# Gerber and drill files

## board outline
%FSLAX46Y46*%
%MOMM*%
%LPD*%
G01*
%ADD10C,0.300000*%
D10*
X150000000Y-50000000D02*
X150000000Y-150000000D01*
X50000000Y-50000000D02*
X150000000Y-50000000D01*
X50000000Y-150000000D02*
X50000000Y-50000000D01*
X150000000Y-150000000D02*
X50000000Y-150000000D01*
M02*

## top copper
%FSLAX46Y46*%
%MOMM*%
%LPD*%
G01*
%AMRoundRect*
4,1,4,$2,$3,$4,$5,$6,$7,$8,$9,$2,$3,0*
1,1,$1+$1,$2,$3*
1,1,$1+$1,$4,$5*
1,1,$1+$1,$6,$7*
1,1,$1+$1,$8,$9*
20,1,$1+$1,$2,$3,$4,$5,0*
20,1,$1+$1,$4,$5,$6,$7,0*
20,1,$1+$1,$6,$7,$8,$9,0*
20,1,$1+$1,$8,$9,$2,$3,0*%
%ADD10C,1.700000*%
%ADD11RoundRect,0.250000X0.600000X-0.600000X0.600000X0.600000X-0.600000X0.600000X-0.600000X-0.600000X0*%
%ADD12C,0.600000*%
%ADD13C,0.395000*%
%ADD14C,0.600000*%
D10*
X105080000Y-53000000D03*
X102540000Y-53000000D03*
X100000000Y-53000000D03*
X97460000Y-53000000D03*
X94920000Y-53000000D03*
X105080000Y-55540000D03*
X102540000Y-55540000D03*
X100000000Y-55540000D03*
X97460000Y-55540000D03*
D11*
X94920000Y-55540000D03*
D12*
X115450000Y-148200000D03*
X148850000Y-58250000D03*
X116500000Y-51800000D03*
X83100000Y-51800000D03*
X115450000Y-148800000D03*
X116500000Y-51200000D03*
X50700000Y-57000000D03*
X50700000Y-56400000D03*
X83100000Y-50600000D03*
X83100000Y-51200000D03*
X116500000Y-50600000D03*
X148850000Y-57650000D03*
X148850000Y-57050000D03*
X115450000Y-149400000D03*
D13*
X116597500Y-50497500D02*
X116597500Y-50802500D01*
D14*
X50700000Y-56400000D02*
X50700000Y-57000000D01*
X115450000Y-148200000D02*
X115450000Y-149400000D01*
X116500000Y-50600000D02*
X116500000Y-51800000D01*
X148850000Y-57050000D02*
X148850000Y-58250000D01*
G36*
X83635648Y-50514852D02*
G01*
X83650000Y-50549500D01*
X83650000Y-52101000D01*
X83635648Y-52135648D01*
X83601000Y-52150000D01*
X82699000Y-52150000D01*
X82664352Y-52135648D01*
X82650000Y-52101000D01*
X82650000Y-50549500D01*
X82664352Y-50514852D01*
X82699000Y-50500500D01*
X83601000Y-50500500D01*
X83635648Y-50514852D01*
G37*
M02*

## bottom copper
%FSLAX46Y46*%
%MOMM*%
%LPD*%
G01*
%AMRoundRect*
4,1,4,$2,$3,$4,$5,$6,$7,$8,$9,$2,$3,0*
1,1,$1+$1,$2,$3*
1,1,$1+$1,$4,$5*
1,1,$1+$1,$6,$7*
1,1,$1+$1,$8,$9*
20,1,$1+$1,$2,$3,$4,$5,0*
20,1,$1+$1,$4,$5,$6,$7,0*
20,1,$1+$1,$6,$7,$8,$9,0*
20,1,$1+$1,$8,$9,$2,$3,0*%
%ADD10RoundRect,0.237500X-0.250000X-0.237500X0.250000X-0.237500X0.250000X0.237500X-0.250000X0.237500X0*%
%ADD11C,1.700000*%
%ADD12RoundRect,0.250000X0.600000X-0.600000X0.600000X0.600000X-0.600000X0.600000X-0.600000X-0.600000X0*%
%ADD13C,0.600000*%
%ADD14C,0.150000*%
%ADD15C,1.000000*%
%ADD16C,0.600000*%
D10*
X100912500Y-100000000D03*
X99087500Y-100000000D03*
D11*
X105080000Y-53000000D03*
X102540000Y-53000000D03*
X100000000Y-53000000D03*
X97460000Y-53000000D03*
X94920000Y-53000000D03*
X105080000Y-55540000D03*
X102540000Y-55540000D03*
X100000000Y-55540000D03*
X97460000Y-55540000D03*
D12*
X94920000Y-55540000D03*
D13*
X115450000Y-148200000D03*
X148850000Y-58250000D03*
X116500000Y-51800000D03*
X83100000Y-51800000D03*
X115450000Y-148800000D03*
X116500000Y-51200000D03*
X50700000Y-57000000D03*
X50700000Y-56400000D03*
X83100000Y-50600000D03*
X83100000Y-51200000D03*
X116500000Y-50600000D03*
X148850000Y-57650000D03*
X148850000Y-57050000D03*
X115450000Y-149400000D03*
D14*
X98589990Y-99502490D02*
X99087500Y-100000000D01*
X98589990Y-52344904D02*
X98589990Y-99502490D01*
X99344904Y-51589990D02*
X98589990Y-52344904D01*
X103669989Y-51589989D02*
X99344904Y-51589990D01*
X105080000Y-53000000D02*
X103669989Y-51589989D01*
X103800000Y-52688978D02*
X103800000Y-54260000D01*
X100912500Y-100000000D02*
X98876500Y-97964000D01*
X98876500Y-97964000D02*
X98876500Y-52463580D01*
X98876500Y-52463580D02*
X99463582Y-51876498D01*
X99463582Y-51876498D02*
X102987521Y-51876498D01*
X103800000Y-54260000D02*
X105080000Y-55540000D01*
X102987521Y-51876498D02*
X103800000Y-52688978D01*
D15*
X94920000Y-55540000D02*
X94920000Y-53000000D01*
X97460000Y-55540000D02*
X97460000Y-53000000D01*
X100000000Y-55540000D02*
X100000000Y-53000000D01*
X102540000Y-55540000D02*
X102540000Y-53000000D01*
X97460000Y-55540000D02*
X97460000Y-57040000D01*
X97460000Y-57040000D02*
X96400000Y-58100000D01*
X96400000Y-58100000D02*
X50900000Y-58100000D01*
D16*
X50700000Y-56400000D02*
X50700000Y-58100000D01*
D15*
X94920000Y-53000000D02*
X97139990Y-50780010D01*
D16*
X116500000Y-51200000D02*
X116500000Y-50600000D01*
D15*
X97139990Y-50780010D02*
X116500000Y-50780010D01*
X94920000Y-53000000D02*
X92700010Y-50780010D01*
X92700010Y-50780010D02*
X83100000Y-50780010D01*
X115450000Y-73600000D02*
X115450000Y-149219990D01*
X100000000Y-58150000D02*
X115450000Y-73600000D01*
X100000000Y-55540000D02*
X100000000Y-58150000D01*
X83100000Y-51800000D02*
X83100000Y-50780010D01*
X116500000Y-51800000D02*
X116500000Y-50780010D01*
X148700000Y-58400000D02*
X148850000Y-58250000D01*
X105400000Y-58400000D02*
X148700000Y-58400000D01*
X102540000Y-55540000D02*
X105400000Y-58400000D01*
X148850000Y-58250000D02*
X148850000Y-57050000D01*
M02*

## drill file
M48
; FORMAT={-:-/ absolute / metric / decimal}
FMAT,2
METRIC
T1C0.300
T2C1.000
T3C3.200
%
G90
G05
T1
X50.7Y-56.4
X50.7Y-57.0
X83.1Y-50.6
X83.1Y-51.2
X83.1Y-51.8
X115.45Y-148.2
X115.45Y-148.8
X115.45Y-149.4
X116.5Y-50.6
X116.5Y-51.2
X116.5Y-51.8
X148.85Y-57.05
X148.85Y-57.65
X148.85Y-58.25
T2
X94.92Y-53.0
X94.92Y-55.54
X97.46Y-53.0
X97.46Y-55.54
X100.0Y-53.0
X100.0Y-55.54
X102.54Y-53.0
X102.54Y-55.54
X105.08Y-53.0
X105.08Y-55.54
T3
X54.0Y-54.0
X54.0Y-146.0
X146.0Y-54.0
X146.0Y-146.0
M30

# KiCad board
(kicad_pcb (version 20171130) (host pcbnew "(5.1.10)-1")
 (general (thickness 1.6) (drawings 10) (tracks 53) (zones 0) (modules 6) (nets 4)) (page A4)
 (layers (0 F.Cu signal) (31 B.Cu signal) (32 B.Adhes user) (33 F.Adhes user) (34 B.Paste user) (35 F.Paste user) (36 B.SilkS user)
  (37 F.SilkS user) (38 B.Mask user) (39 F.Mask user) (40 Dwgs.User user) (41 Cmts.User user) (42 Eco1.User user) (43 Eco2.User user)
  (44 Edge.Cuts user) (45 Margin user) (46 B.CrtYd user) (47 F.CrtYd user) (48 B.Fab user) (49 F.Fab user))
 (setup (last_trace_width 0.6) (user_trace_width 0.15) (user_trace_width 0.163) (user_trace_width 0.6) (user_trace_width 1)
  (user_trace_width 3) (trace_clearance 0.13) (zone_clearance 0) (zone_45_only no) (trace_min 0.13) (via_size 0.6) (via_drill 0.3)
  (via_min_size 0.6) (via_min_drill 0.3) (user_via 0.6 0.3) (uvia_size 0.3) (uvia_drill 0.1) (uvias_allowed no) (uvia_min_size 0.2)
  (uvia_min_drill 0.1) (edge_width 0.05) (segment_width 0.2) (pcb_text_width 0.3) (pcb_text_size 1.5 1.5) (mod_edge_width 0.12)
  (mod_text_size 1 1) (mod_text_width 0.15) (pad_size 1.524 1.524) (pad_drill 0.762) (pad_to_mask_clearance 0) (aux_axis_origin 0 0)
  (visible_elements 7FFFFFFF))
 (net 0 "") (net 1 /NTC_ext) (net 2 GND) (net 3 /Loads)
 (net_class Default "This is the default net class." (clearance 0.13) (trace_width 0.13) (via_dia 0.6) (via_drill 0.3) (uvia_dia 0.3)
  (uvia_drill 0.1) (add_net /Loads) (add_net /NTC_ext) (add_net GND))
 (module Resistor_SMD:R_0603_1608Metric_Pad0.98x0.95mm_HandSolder (layer B.Cu) (at 100 100)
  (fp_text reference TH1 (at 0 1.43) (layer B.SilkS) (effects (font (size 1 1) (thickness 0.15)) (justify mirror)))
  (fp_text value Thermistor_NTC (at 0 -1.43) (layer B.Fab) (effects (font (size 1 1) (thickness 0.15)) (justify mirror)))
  (pad 2 smd roundrect (at 0.9125 0) (size 0.975 0.95) (layers B.Cu B.Paste B.Mask) (roundrect_rratio 0.25) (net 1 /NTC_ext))
  (pad 1 smd roundrect (at -0.9125 0) (size 0.975 0.95) (layers B.Cu B.Paste B.Mask) (roundrect_rratio 0.25) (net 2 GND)))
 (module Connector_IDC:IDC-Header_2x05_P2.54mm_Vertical (layer F.Cu) (at 94.92 55.54 90)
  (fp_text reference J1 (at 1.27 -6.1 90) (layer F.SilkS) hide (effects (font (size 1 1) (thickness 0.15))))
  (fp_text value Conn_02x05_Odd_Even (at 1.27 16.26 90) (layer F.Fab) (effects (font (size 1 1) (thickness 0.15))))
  (pad 10 thru_hole circle (at 2.54 10.16 90) (size 1.7 1.7) (drill 1) (layers *.Cu *.Mask) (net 2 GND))
  (pad 8 thru_hole circle (at 2.54 7.62 90) (size 1.7 1.7) (drill 1) (layers *.Cu *.Mask) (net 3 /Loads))
  (pad 6 thru_hole circle (at 2.54 5.08 90) (size 1.7 1.7) (drill 1) (layers *.Cu *.Mask) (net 3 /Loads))
  (pad 4 thru_hole circle (at 2.54 2.54 90) (size 1.7 1.7) (drill 1) (layers *.Cu *.Mask) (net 3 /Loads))
  (pad 2 thru_hole circle (at 2.54 0 90) (size 1.7 1.7) (drill 1) (layers *.Cu *.Mask) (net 3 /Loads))
  (pad 9 thru_hole circle (at 0 10.16 90) (size 1.7 1.7) (drill 1) (layers *.Cu *.Mask) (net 1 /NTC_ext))
  (pad 7 thru_hole circle (at 0 7.62 90) (size 1.7 1.7) (drill 1) (layers *.Cu *.Mask) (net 3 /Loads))
  (pad 5 thru_hole circle (at 0 5.08 90) (size 1.7 1.7) (drill 1) (layers *.Cu *.Mask) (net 3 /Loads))
  (pad 3 thru_hole circle (at 0 2.54 90) (size 1.7 1.7) (drill 1) (layers *.Cu *.Mask) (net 3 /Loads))
  (pad 1 thru_hole roundrect (at 0 0 90) (size 1.7 1.7) (drill 1) (layers *.Cu *.Mask) (roundrect_rratio 0.1470588235294118) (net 3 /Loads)))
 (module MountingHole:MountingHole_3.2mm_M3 (layer F.Cu) (at 146 146)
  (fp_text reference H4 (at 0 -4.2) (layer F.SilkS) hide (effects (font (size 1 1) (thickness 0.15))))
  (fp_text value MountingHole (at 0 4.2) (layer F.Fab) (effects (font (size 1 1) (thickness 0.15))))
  (pad 1 np_thru_hole circle (at 0 0) (size 3.2 3.2) (drill 3.2) (layers *.Cu *.Mask)))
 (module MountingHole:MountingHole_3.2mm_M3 (layer F.Cu) (at 54 146)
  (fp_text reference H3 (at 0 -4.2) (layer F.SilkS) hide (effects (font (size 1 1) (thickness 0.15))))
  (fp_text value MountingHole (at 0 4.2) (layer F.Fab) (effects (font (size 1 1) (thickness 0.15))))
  (pad 1 np_thru_hole circle (at 0 0) (size 3.2 3.2) (drill 3.2) (layers *.Cu *.Mask)))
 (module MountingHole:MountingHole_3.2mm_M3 (layer F.Cu) (at 146 54)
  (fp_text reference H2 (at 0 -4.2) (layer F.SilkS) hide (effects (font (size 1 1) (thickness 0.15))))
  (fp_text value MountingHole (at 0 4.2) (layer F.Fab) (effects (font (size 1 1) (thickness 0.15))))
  (pad 1 np_thru_hole circle (at 0 0) (size 3.2 3.2) (drill 3.2) (layers *.Cu *.Mask)))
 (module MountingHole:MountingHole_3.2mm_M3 (layer F.Cu) (at 54 54)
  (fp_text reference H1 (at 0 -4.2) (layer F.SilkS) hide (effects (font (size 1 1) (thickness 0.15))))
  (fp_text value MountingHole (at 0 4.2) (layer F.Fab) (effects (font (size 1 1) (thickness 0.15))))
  (pad 1 np_thru_hole circle (at 0 0) (size 3.2 3.2) (drill 3.2) (layers *.Cu *.Mask)))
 (gr_line (start 150 50) (end 150 150) (layer Edge.Cuts) (width 0.3))
 (gr_line (start 50 50) (end 150 50) (layer Edge.Cuts) (width 0.3))
 (gr_line (start 50 150) (end 50 50) (layer Edge.Cuts) (width 0.3))
 (gr_line (start 150 150) (end 50 150) (layer Edge.Cuts) (width 0.3))
 (segment (start 98.58999 99.50249) (end 99.0875 100) (width 0.15) (layer B.Cu) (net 2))
 (segment (start 98.58999 52.344904) (end 98.58999 99.50249) (width 0.15) (layer B.Cu) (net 2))
 (segment (start 99.344904 51.58999) (end 98.58999 52.344904) (width 0.15) (layer B.Cu) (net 2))
 (segment (start 103.669989 51.589989) (end 99.344904 51.58999) (width 0.15) (layer B.Cu) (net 2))
 (segment (start 105.08 53) (end 103.669989 51.589989) (width 0.15) (layer B.Cu) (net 2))
 (segment (start 103.8 52.688978) (end 103.8 54.26) (width 0.15) (layer B.Cu) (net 1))
 (segment (start 100.9125 100) (end 98.8765 97.964) (width 0.15) (layer B.Cu) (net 1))
 (segment (start 98.8765 97.964) (end 98.8765 52.46358) (width 0.15) (layer B.Cu) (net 1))
 (segment (start 98.8765 52.46358) (end 99.463582 51.876498) (width 0.15) (layer B.Cu) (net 1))
 (segment (start 99.463582 51.876498) (end 102.987521 51.876498) (width 0.15) (layer B.Cu) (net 1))
 (segment (start 103.8 54.26) (end 105.08 55.54) (width 0.15) (layer B.Cu) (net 1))
 (segment (start 102.987521 51.876498) (end 103.8 52.688978) (width 0.15) (layer B.Cu) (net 1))
 (via (at 115.45 148.2) (size 0.6) (drill 0.3) (layers F.Cu B.Cu) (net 3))
 (via (at 148.85 58.25) (size 0.6) (drill 0.3) (layers F.Cu B.Cu) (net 3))
 (via (at 116.5 51.8) (size 0.6) (drill 0.3) (layers F.Cu B.Cu) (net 3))
 (via (at 83.1 51.8) (size 0.6) (drill 0.3) (layers F.Cu B.Cu) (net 3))
 (via (at 115.45 148.8) (size 0.6) (drill 0.3) (layers F.Cu B.Cu) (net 3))
 (via (at 116.5 51.2) (size 0.6) (drill 0.3) (layers F.Cu B.Cu) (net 3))
 (via (at 50.7 57) (size 0.6) (drill 0.3) (layers F.Cu B.Cu) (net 3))
 (via (at 50.7 56.4) (size 0.6) (drill 0.3) (layers F.Cu B.Cu) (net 3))
 (segment (start 94.92 55.54) (end 94.92 53) (width 1) (layer B.Cu) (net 3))
 (segment (start 97.46 55.54) (end 97.46 53) (width 1) (layer B.Cu) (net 3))
 (segment (start 100 55.54) (end 100 53) (width 1) (layer B.Cu) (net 3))
 (segment (start 102.54 55.54) (end 102.54 53) (width 1) (layer B.Cu) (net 3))
 (segment (start 116.5975 50.4975) (end 116.5975 50.8025) (width 0.395) (layer F.Cu) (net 3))
 (via (at 83.1 50.6) (size 0.6) (drill 0.3) (layers F.Cu B.Cu) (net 3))
 (via (at 83.1 51.2) (size 0.6) (drill 0.3) (layers F.Cu B.Cu) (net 3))
 (segment (start 97.46 55.54) (end 97.46 57.04) (width 1) (layer B.Cu) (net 3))
 (segment (start 97.46 57.04) (end 96.4 58.1) (width 1) (layer B.Cu) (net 3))
 (segment (start 96.4 58.1) (end 50.9 58.1) (width 1) (layer B.Cu) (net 3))
 (segment (start 50.7 56.4) (end 50.7 58.1) (width 0.6) (layer B.Cu) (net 3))
 (segment (start 50.7 56.4) (end 50.7 57) (width 0.6) (layer F.Cu) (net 3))
 (via (at 116.5 50.6) (size 0.6) (drill 0.3) (layers F.Cu B.Cu) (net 3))
 (segment (start 94.92 53) (end 97.13999 50.78001) (width 1) (layer B.Cu) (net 3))
 (segment (start 116.5 51.2) (end 116.5 50.6) (width 0.6) (layer B.Cu) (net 3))
 (segment (start 97.13999 50.78001) (end 116.5 50.78001) (width 1) (layer B.Cu) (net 3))
 (segment (start 94.92 53) (end 92.70001 50.78001) (width 1) (layer B.Cu) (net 3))
 (segment (start 92.70001 50.78001) (end 83.1 50.78001) (width 1) (layer B.Cu) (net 3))
 (via (at 148.85 57.65) (size 0.6) (drill 0.3) (layers F.Cu B.Cu) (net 3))
 (via (at 148.85 57.05) (size 0.6) (drill 0.3) (layers F.Cu B.Cu) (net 3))
 (via (at 115.45 149.4) (size 0.6) (drill 0.3) (layers F.Cu B.Cu) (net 3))
 (segment (start 115.45 73.6) (end 115.45 149.21999) (width 1) (layer B.Cu) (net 3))
 (segment (start 100 58.15) (end 115.45 73.6) (width 1) (layer B.Cu) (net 3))
 (segment (start 100 55.54) (end 100 58.15) (width 1) (layer B.Cu) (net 3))
 (segment (start 83.1 51.8) (end 83.1 50.78001) (width 1) (layer B.Cu) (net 3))
 (segment (start 116.5 51.8) (end 116.5 50.78001) (width 1) (layer B.Cu) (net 3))
 (segment (start 148.7 58.4) (end 148.85 58.25) (width 1) (layer B.Cu) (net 3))
 (segment (start 105.4 58.4) (end 148.7 58.4) (width 1) (layer B.Cu) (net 3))
 (segment (start 102.54 55.54) (end 105.4 58.4) (width 1) (layer B.Cu) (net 3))
 (segment (start 115.45 148.2) (end 115.45 149.4) (width 0.6) (layer F.Cu) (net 3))
 (segment (start 116.5 50.6) (end 116.5 51.8) (width 0.6) (layer F.Cu) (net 3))
 (segment (start 148.85 58.25) (end 148.85 57.05) (width 1) (layer B.Cu) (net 3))
 (segment (start 148.85 57.05) (end 148.85 58.25) (width 0.6) (layer F.Cu) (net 3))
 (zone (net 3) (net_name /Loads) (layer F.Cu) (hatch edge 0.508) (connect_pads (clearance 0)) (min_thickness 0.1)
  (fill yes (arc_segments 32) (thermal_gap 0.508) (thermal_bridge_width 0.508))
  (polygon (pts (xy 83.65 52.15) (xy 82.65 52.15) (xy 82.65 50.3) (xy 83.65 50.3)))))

